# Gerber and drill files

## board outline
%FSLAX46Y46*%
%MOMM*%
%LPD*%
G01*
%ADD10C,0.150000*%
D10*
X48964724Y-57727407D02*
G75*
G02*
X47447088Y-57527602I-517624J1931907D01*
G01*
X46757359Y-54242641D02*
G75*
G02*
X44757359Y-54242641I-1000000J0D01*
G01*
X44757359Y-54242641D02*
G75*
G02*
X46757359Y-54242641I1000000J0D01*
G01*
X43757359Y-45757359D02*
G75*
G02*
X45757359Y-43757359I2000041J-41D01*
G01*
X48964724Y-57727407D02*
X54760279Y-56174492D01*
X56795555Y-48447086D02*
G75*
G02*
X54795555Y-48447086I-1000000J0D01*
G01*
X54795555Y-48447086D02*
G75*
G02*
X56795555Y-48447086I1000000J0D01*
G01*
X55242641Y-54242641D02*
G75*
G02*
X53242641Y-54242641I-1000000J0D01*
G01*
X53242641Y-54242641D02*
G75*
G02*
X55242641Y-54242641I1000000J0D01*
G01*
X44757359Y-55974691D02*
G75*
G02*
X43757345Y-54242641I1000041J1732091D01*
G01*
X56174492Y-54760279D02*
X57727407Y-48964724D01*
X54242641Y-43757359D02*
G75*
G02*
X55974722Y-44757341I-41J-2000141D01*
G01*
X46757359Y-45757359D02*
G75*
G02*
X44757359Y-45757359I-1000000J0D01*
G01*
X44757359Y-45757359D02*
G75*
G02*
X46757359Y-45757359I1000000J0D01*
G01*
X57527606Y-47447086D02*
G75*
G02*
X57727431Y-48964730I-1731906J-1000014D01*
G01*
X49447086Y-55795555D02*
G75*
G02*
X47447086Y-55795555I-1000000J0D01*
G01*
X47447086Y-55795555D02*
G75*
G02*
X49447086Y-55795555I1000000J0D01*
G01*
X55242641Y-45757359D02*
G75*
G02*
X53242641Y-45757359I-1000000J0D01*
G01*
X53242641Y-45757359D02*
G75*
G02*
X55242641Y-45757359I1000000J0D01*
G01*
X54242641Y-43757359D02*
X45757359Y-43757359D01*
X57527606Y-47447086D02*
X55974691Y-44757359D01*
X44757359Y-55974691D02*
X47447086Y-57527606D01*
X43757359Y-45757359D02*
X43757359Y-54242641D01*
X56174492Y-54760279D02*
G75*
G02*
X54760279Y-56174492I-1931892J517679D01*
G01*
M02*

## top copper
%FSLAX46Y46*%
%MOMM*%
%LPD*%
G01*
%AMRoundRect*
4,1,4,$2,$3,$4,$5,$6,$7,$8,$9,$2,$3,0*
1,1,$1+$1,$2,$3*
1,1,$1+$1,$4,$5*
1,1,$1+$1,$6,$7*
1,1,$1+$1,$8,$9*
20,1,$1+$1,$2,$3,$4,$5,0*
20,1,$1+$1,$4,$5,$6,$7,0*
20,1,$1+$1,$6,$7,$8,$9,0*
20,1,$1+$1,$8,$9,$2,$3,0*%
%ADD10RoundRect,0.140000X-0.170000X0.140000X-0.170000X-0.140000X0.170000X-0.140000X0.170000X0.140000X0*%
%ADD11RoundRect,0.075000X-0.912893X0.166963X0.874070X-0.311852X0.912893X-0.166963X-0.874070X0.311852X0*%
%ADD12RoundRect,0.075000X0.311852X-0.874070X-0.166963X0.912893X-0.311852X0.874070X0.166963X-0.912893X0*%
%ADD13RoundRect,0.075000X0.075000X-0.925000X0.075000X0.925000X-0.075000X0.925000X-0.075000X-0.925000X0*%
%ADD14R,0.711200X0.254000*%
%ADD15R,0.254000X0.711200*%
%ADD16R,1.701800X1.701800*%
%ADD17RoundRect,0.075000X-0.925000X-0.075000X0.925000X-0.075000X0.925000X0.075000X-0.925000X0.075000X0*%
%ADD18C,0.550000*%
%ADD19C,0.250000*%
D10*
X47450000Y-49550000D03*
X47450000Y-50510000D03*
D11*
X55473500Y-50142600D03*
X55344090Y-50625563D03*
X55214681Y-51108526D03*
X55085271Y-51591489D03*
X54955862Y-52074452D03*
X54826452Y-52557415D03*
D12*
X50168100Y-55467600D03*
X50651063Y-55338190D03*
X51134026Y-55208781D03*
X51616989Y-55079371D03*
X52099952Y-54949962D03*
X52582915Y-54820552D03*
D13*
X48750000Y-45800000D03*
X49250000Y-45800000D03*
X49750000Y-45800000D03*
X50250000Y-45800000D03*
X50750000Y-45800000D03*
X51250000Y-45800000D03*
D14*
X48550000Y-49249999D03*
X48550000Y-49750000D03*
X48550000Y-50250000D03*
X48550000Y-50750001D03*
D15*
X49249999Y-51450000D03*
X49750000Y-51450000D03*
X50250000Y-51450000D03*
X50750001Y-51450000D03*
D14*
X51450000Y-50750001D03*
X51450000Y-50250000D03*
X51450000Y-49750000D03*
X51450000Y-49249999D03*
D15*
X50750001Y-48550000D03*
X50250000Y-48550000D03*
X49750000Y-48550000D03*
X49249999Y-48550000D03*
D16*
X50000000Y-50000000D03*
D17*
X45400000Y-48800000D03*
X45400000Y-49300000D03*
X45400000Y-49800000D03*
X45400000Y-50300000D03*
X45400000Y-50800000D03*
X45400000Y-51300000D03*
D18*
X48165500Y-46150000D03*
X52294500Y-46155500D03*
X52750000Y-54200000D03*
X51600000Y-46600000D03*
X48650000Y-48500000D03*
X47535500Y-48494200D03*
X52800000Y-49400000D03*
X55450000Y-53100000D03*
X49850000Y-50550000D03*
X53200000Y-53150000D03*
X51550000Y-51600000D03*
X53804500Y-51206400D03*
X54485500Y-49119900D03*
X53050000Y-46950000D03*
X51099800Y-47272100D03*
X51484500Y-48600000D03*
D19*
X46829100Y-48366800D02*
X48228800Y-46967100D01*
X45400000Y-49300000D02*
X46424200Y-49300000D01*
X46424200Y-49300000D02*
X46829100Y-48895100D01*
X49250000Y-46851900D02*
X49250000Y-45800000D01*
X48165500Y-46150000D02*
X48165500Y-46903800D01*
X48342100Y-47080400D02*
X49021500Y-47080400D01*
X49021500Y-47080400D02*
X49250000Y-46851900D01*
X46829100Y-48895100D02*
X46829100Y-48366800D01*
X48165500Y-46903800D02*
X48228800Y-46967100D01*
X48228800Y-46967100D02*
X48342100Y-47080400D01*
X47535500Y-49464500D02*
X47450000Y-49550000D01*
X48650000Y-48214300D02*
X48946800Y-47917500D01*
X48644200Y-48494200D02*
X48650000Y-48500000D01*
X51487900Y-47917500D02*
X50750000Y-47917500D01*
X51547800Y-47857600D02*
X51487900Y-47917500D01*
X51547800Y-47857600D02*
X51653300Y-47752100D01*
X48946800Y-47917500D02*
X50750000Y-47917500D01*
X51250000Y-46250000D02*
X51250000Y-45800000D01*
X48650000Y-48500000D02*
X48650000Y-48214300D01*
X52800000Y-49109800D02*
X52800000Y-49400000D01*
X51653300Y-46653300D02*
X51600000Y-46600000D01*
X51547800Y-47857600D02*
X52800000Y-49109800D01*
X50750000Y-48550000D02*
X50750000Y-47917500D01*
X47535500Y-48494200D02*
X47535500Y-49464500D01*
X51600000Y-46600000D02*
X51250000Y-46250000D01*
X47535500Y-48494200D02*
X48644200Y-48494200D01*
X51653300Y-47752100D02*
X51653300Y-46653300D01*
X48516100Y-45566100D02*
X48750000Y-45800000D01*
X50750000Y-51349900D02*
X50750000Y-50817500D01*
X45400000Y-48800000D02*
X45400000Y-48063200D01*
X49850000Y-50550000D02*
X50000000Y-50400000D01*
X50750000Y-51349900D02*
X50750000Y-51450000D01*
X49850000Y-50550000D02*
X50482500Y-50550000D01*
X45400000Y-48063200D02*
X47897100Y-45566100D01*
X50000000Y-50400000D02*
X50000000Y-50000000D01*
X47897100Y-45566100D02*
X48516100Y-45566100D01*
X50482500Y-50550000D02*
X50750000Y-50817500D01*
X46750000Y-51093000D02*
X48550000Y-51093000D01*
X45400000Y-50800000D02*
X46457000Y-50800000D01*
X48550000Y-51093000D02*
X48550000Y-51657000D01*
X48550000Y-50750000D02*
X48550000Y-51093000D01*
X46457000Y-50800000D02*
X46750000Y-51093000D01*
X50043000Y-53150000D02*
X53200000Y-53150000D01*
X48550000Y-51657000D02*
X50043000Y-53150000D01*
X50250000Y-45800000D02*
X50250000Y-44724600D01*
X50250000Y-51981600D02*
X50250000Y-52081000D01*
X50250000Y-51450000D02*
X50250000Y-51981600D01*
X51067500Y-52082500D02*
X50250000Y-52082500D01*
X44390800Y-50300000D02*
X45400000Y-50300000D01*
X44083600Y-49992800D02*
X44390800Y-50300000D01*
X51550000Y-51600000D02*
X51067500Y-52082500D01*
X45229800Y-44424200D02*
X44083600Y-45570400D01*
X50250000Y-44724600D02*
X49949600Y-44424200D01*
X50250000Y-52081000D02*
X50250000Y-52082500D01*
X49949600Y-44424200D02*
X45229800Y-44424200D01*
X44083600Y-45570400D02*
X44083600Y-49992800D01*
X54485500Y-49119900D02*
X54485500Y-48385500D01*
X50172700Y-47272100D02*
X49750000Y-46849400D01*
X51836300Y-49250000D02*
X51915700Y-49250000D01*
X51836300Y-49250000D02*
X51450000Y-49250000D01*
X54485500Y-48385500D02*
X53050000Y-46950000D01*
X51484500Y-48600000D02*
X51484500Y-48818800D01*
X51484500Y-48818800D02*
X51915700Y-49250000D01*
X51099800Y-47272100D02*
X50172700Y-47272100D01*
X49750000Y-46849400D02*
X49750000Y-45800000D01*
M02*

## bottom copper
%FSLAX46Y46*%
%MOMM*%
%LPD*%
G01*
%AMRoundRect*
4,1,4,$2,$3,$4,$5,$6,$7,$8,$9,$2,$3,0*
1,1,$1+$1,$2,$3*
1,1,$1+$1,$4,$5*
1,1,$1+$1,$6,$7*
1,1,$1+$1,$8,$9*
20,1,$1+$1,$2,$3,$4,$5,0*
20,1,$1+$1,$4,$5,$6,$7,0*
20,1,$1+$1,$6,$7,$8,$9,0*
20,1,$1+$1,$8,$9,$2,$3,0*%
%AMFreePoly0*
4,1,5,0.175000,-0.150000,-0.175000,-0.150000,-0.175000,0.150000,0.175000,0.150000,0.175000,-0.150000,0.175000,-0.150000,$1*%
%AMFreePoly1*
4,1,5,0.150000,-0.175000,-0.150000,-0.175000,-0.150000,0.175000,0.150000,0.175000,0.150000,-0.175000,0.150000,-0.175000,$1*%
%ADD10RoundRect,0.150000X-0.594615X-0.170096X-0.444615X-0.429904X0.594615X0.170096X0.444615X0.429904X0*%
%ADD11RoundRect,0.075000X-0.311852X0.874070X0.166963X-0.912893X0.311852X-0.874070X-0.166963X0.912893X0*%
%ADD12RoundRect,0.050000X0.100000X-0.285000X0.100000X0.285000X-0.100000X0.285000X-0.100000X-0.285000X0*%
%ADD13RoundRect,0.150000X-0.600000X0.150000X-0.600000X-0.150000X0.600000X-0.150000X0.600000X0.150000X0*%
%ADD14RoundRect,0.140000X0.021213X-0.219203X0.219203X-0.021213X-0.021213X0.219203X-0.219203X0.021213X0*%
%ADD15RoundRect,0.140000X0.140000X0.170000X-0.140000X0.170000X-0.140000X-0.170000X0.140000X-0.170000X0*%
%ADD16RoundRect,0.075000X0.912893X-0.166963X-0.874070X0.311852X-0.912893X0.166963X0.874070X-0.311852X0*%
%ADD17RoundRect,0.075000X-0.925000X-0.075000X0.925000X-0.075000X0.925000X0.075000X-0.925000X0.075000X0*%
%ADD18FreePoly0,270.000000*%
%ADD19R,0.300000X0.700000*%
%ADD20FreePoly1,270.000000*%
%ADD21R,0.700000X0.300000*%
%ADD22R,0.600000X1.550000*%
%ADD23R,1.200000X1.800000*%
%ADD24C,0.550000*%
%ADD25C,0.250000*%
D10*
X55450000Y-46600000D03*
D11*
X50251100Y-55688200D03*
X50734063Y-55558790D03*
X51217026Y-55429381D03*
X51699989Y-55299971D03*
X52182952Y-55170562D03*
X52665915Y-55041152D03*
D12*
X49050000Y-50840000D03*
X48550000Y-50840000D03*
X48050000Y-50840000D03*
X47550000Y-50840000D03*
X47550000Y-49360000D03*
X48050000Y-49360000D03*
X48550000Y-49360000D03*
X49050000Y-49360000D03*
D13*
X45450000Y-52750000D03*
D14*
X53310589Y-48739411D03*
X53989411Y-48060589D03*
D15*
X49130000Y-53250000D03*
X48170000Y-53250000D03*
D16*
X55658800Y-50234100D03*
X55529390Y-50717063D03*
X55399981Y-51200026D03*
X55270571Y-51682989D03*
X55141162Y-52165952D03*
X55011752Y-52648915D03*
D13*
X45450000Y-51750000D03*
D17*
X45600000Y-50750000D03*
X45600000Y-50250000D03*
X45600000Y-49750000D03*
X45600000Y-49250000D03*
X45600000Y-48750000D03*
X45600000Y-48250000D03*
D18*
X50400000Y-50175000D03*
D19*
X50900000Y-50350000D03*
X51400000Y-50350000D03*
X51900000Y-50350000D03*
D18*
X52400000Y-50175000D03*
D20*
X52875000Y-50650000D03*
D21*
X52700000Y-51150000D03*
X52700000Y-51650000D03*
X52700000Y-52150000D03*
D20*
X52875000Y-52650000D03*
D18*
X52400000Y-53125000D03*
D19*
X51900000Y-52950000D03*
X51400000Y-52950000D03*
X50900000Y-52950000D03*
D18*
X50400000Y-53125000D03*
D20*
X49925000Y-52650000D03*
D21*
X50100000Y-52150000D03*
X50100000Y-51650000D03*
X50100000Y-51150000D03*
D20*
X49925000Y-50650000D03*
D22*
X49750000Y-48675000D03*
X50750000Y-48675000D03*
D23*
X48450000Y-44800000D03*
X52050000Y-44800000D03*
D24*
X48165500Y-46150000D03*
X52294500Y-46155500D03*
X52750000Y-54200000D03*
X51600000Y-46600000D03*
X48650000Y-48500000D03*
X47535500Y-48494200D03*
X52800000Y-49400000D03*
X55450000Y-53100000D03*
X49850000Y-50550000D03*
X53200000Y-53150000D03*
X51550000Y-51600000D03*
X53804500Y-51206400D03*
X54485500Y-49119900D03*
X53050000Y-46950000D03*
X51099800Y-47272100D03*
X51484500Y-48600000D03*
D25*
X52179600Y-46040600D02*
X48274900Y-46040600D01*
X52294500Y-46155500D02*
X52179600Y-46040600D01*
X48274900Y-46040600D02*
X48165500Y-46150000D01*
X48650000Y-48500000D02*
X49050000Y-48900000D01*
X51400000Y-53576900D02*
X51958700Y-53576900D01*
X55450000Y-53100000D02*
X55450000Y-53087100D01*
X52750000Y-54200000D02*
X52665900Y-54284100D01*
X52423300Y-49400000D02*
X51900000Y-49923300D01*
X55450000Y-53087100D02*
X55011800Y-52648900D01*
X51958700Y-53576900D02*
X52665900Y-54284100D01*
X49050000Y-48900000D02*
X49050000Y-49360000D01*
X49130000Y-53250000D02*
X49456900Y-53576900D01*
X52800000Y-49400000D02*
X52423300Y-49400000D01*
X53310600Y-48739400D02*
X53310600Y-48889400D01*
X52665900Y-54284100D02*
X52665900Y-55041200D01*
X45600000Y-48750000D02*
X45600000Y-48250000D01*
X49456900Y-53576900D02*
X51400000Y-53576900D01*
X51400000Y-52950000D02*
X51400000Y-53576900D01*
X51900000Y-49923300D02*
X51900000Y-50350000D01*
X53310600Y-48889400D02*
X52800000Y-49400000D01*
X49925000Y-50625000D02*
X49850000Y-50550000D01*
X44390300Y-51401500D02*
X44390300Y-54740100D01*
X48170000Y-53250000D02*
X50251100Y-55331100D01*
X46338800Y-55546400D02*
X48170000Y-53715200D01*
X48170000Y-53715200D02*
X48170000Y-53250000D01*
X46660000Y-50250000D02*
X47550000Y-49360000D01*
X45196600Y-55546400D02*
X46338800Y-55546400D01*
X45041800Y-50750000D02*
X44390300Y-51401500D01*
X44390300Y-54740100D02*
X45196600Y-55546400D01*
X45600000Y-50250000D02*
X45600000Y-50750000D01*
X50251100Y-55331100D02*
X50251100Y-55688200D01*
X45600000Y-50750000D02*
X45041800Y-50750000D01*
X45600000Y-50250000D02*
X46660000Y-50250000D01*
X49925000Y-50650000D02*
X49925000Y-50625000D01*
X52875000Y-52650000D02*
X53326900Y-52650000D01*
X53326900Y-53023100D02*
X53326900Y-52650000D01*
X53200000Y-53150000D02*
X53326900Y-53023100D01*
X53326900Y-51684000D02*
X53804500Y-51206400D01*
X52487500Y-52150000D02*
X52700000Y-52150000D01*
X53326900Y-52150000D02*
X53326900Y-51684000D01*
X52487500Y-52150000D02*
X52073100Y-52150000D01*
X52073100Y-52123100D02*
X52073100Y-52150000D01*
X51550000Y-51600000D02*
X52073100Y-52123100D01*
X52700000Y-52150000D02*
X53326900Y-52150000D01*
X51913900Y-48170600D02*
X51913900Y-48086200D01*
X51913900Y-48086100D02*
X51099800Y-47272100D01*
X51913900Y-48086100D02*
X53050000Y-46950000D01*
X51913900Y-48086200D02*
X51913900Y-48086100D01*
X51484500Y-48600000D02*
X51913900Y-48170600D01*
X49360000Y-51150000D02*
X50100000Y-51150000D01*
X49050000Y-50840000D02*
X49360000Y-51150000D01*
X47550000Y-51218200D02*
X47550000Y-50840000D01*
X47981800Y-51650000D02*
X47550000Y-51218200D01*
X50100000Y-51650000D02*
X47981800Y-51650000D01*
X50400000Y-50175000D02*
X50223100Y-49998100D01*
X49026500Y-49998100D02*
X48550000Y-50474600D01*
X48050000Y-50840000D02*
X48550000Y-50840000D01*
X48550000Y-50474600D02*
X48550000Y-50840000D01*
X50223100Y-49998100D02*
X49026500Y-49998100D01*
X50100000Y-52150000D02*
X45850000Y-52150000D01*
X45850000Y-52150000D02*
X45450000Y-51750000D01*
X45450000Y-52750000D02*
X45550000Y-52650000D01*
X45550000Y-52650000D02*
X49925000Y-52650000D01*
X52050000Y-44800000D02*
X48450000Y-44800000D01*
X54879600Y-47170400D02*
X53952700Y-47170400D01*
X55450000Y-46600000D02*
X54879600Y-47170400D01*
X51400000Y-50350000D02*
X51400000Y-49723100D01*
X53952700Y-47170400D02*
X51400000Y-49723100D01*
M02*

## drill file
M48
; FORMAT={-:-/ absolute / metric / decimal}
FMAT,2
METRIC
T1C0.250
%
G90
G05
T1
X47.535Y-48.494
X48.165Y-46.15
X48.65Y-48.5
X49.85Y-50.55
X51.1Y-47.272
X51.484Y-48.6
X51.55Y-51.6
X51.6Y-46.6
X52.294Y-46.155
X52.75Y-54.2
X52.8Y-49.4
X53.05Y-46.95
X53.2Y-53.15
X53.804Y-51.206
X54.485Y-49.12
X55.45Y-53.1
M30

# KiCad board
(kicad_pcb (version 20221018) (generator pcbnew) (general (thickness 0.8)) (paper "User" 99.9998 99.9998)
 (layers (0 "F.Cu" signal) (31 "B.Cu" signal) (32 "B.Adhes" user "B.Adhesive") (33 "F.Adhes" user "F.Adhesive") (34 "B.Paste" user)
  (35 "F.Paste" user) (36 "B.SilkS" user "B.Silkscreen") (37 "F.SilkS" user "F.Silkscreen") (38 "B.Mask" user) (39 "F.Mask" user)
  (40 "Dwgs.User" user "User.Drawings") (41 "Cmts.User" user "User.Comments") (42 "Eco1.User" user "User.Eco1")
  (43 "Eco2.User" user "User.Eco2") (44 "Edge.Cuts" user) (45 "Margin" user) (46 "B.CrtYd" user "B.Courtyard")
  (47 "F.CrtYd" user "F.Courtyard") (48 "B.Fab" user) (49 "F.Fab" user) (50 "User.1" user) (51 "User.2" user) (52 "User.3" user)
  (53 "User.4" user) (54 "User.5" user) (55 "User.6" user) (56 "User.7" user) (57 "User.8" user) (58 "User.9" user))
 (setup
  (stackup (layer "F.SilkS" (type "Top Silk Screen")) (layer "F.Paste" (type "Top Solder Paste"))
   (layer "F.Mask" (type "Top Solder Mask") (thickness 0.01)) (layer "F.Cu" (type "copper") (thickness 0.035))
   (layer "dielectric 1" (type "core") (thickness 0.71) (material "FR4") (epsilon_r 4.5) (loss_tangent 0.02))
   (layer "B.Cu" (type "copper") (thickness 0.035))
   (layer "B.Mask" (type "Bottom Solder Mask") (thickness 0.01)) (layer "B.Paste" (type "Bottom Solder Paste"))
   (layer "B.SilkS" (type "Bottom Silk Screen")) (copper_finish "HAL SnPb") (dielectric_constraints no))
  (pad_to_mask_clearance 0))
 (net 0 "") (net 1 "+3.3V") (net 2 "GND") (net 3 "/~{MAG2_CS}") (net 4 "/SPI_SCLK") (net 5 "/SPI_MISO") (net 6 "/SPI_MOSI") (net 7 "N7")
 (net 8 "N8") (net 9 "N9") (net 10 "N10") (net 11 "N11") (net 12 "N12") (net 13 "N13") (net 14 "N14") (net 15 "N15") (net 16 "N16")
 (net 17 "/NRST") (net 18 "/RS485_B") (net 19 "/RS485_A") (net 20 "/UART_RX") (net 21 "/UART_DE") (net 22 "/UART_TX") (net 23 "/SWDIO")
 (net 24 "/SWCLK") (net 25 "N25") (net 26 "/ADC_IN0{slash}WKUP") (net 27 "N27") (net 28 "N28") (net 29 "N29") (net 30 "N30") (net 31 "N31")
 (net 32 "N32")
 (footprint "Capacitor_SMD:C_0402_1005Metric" (layer "F.Cu") (at 47.45 50.03 -90)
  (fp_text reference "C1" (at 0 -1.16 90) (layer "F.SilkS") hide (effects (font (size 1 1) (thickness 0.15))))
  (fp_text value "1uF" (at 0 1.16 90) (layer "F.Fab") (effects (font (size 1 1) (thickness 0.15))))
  (pad "1" smd roundrect (at -0.48 0 270) (size 0.56 0.62) (layers "F.Cu" "F.Paste" "F.Mask") (roundrect_rratio 0.25) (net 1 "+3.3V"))
  (pad "2" smd roundrect (at 0.48 0 270) (size 0.56 0.62) (layers "F.Cu" "F.Paste" "F.Mask") (roundrect_rratio 0.25) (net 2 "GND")))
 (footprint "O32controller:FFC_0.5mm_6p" (layer "F.Cu") (at 55.4735 50.1426 -15)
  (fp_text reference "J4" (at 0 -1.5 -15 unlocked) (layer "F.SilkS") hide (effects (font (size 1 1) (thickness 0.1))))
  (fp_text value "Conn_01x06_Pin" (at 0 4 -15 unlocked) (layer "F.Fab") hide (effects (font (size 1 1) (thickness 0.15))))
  (pad "1" smd roundrect (at 0 0 345) (size 2 0.3) (layers "F.Cu" "F.Mask") (roundrect_rratio 0.25) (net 2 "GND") (thermal_bridge_angle 45))
  (pad "2" smd roundrect (at 0 0.5 345) (size 2 0.3) (layers "F.Cu" "F.Mask") (roundrect_rratio 0.25) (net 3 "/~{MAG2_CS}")
   (thermal_bridge_angle 45))
  (pad "3" smd roundrect (at 0 1 345) (size 2 0.3) (layers "F.Cu" "F.Mask") (roundrect_rratio 0.25) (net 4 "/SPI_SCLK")
   (thermal_bridge_angle 45))
  (pad "4" smd roundrect (at 0 1.5 345) (size 2 0.3) (layers "F.Cu" "F.Mask") (roundrect_rratio 0.25) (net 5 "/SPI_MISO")
   (thermal_bridge_angle 45))
  (pad "5" smd roundrect (at 0 2 345) (size 2 0.3) (layers "F.Cu" "F.Mask") (roundrect_rratio 0.25) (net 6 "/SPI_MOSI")
   (thermal_bridge_angle 45))
  (pad "6" smd roundrect (at 0 2.5 345) (size 2 0.3) (layers "F.Cu" "F.Mask") (roundrect_rratio 0.25) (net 1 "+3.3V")
   (thermal_bridge_angle 45)))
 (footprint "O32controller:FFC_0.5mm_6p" (layer "F.Cu") (at 50.1681 55.4676 105)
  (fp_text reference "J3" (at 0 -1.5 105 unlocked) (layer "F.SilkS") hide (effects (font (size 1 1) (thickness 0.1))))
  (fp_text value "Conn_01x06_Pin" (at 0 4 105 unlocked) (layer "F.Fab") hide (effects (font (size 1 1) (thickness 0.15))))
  (pad "1" smd roundrect (at 0 0 105) (size 2 0.3) (layers "F.Cu" "F.Mask") (roundrect_rratio 0.25) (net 2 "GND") (thermal_bridge_angle 45))
  (pad "2" smd roundrect (at 0 0.5 105) (size 2 0.3) (layers "F.Cu" "F.Mask") (roundrect_rratio 0.25) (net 3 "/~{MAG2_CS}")
   (thermal_bridge_angle 45))
  (pad "3" smd roundrect (at 0 1 105) (size 2 0.3) (layers "F.Cu" "F.Mask") (roundrect_rratio 0.25) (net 4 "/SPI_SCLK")
   (thermal_bridge_angle 45))
  (pad "4" smd roundrect (at 0 1.5 105) (size 2 0.3) (layers "F.Cu" "F.Mask") (roundrect_rratio 0.25) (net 5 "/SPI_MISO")
   (thermal_bridge_angle 45))
  (pad "5" smd roundrect (at 0 2 105) (size 2 0.3) (layers "F.Cu" "F.Mask") (roundrect_rratio 0.25) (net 6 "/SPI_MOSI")
   (thermal_bridge_angle 45))
  (pad "6" smd roundrect (at 0 2.5 105) (size 2 0.3) (layers "F.Cu" "F.Mask") (roundrect_rratio 0.25) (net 1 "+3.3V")
   (thermal_bridge_angle 45)))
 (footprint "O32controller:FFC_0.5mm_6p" (layer "F.Cu") (at 48.75 45.8 90)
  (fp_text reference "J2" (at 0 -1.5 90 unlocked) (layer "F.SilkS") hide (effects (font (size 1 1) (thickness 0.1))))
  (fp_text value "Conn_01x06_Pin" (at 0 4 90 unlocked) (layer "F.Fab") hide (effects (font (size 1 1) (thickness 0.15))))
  (pad "1" smd roundrect (at 0 0 90) (size 2 0.3) (layers "F.Cu" "F.Mask") (roundrect_rratio 0.25) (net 2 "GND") (thermal_bridge_angle 45))
  (pad "2" smd roundrect (at 0 0.5 90) (size 2 0.3) (layers "F.Cu" "F.Mask") (roundrect_rratio 0.25) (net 3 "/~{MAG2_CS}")
   (thermal_bridge_angle 45))
  (pad "3" smd roundrect (at 0 1 90) (size 2 0.3) (layers "F.Cu" "F.Mask") (roundrect_rratio 0.25) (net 4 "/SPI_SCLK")
   (thermal_bridge_angle 45))
  (pad "4" smd roundrect (at 0 1.5 90) (size 2 0.3) (layers "F.Cu" "F.Mask") (roundrect_rratio 0.25) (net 5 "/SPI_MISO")
   (thermal_bridge_angle 45))
  (pad "5" smd roundrect (at 0 2 90) (size 2 0.3) (layers "F.Cu" "F.Mask") (roundrect_rratio 0.25) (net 6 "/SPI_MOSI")
   (thermal_bridge_angle 45))
  (pad "6" smd roundrect (at 0 2.5 90) (size 2 0.3) (layers "F.Cu" "F.Mask") (roundrect_rratio 0.25) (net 1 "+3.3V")
   (thermal_bridge_angle 45)))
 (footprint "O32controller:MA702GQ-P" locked (layer "F.Cu") (at 50 50)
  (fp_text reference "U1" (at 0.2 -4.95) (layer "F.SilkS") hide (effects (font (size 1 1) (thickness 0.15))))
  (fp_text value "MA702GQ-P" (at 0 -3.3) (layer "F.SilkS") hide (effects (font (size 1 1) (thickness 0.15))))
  (pad "1" smd rect locked (at -1.45 -0.750001) (size 0.7112 0.254) (layers "F.Cu" "F.Paste" "F.Mask") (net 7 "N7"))
  (pad "2" smd rect locked (at -1.45 -0.25) (size 0.7112 0.254) (layers "F.Cu" "F.Paste" "F.Mask") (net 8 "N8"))
  (pad "3" smd rect locked (at -1.45 0.25) (size 0.7112 0.254) (layers "F.Cu" "F.Paste" "F.Mask") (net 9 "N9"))
  (pad "4" smd rect locked (at -1.45 0.750001) (size 0.7112 0.254) (layers "F.Cu" "F.Paste" "F.Mask") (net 6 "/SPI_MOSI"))
  (pad "5" smd rect locked (at -0.750001 1.45 90) (size 0.7112 0.254) (layers "F.Cu" "F.Paste" "F.Mask") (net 3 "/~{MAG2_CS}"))
  (pad "6" smd rect locked (at -0.25 1.45 90) (size 0.7112 0.254) (layers "F.Cu" "F.Paste" "F.Mask") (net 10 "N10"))
  (pad "7" smd rect locked (at 0.25 1.45 90) (size 0.7112 0.254) (layers "F.Cu" "F.Paste" "F.Mask") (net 5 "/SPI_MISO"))
  (pad "8" smd rect locked (at 0.750001 1.45 90) (size 0.7112 0.254) (layers "F.Cu" "F.Paste" "F.Mask") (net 2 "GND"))
  (pad "9" smd rect locked (at 1.45 0.750001) (size 0.7112 0.254) (layers "F.Cu" "F.Paste" "F.Mask") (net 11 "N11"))
  (pad "10" smd rect locked (at 1.45 0.25) (size 0.7112 0.254) (layers "F.Cu" "F.Paste" "F.Mask") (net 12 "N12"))
  (pad "11" smd rect locked (at 1.45 -0.25) (size 0.7112 0.254) (layers "F.Cu" "F.Paste" "F.Mask") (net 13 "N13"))
  (pad "12" smd rect locked (at 1.45 -0.750001) (size 0.7112 0.254) (layers "F.Cu" "F.Paste" "F.Mask") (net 4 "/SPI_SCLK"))
  (pad "13" smd rect locked (at 0.750001 -1.45 90) (size 0.7112 0.254) (layers "F.Cu" "F.Paste" "F.Mask") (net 1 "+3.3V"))
  (pad "14" smd rect locked (at 0.25 -1.45 90) (size 0.7112 0.254) (layers "F.Cu" "F.Paste" "F.Mask") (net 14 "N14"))
  (pad "15" smd rect locked (at -0.25 -1.45 90) (size 0.7112 0.254) (layers "F.Cu" "F.Paste" "F.Mask") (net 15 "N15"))
  (pad "16" smd rect locked (at -0.750001 -1.45 90) (size 0.7112 0.254) (layers "F.Cu" "F.Paste" "F.Mask") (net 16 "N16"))
  (pad "17" smd rect locked (at 0 0) (size 1.7018 1.7018) (layers "F.Cu" "F.Paste" "F.Mask") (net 2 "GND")))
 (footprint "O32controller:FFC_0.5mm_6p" (layer "F.Cu") (at 45.4 48.8)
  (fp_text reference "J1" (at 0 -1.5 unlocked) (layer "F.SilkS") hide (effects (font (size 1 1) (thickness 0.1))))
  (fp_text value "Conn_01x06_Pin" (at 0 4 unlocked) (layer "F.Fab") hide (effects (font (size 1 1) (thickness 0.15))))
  (pad "1" smd roundrect (at 0 0) (size 2 0.3) (layers "F.Cu" "F.Mask") (roundrect_rratio 0.25) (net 2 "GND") (thermal_bridge_angle 45))
  (pad "2" smd roundrect (at 0 0.5) (size 2 0.3) (layers "F.Cu" "F.Mask") (roundrect_rratio 0.25) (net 3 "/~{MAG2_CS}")
   (thermal_bridge_angle 45))
  (pad "3" smd roundrect (at 0 1) (size 2 0.3) (layers "F.Cu" "F.Mask") (roundrect_rratio 0.25) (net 4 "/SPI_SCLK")
   (thermal_bridge_angle 45))
  (pad "4" smd roundrect (at 0 1.5) (size 2 0.3) (layers "F.Cu" "F.Mask") (roundrect_rratio 0.25) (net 5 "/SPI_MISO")
   (thermal_bridge_angle 45))
  (pad "5" smd roundrect (at 0 2) (size 2 0.3) (layers "F.Cu" "F.Mask") (roundrect_rratio 0.25) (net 6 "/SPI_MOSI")
   (thermal_bridge_angle 45))
  (pad "6" smd roundrect (at 0 2.5) (size 2 0.3) (layers "F.Cu" "F.Mask") (roundrect_rratio 0.25) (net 1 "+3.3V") (thermal_bridge_angle 45)))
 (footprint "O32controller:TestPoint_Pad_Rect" (layer "B.Cu") (at 55.45 46.6 -60)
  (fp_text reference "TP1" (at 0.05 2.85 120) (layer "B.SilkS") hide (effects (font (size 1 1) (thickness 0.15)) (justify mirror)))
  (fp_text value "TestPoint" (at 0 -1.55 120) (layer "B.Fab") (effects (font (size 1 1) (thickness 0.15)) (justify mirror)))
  (pad "1" smd roundrect (at 0 0 300) (size 0.6 1.5) (layers "B.Cu" "B.Mask") (roundrect_rratio 0.25) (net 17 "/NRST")))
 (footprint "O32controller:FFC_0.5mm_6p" (layer "B.Cu") (at 50.2511 55.6882 -75)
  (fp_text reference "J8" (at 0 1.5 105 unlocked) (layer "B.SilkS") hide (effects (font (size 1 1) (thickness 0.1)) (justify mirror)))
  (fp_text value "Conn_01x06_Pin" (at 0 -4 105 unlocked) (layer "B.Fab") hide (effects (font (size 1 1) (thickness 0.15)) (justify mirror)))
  (pad "1" smd roundrect (at 0 0 285) (size 2 0.3) (layers "B.Cu" "B.Mask") (roundrect_rratio 0.25) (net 2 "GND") (thermal_bridge_angle 45))
  (pad "2" smd roundrect (at 0 -0.5 285) (size 2 0.3) (layers "B.Cu" "B.Mask") (roundrect_rratio 0.25) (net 2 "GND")
   (thermal_bridge_angle 45))
  (pad "3" smd roundrect (at 0 -1 285) (size 2 0.3) (layers "B.Cu" "B.Mask") (roundrect_rratio 0.25) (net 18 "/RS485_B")
   (thermal_bridge_angle 45))
  (pad "4" smd roundrect (at 0 -1.5 285) (size 2 0.3) (layers "B.Cu" "B.Mask") (roundrect_rratio 0.25) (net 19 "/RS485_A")
   (thermal_bridge_angle 45))
  (pad "5" smd roundrect (at 0 -2 285) (size 2 0.3) (layers "B.Cu" "B.Mask") (roundrect_rratio 0.25) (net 1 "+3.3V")
   (thermal_bridge_angle 45))
  (pad "6" smd roundrect (at 0 -2.5 285) (size 2 0.3) (layers "B.Cu" "B.Mask") (roundrect_rratio 0.25) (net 1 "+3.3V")
   (thermal_bridge_angle 45)))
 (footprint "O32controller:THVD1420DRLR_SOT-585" (layer "B.Cu") (at 48.3 50.1 90)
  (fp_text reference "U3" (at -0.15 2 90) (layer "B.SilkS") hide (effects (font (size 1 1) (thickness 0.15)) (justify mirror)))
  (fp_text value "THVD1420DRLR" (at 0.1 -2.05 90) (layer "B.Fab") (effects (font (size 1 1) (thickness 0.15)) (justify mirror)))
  (pad "1" smd roundrect (at -0.74 0.75 90) (size 0.67 0.3) (layers "B.Cu" "B.Paste" "B.Mask") (roundrect_rratio 0.1666666667)
   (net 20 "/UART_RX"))
  (pad "2" smd roundrect (at -0.74 0.25 90) (size 0.67 0.3) (layers "B.Cu" "B.Paste" "B.Mask") (roundrect_rratio 0.1666666667)
   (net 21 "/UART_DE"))
  (pad "3" smd roundrect (at -0.74 -0.25 90) (size 0.67 0.3) (layers "B.Cu" "B.Paste" "B.Mask") (roundrect_rratio 0.1666666667)
   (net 21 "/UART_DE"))
  (pad "4" smd roundrect (at -0.74 -0.75 90) (size 0.67 0.3) (layers "B.Cu" "B.Paste" "B.Mask") (roundrect_rratio 0.1666666667)
   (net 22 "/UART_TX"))
  (pad "5" smd roundrect (at 0.74 -0.75 90) (size 0.67 0.3) (layers "B.Cu" "B.Paste" "B.Mask") (roundrect_rratio 0.1666666667) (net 2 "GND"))
  (pad "6" smd roundrect (at 0.74 -0.25 90) (size 0.67 0.3) (layers "B.Cu" "B.Paste" "B.Mask") (roundrect_rratio 0.1666666667)
   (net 19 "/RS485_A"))
  (pad "7" smd roundrect (at 0.74 0.25 90) (size 0.67 0.3) (layers "B.Cu" "B.Paste" "B.Mask") (roundrect_rratio 0.1666666667)
   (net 18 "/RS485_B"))
  (pad "8" smd roundrect (at 0.74 0.75 90) (size 0.67 0.3) (layers "B.Cu" "B.Paste" "B.Mask") (roundrect_rratio 0.1666666667)
   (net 1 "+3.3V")))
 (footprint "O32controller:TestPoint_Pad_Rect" (layer "B.Cu") (at 45.45 52.75 -90)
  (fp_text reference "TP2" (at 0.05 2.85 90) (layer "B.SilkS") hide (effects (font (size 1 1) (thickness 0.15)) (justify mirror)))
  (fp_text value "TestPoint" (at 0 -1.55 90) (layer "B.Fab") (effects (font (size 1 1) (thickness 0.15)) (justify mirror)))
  (pad "1" smd roundrect (at 0 0 270) (size 0.6 1.5) (layers "B.Cu" "B.Mask") (roundrect_rratio 0.25) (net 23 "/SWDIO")))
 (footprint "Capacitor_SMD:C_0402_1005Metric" (layer "B.Cu") (at 53.65 48.4 45)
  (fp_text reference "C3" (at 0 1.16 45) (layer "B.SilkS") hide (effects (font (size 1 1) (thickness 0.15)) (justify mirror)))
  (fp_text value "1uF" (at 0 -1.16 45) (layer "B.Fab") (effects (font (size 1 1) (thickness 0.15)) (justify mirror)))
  (pad "1" smd roundrect (at -0.48 0 45) (size 0.56 0.62) (layers "B.Cu" "B.Paste" "B.Mask") (roundrect_rratio 0.25) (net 1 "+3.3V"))
  (pad "2" smd roundrect (at 0.48 0 45) (size 0.56 0.62) (layers "B.Cu" "B.Paste" "B.Mask") (roundrect_rratio 0.25) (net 2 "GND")))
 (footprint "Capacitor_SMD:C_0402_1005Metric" (layer "B.Cu") (at 48.65 53.25 180)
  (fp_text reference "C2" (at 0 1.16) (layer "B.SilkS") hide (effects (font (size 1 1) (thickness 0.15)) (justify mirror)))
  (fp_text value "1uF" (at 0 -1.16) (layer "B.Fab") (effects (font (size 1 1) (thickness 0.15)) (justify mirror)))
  (pad "1" smd roundrect (at -0.48 0 180) (size 0.56 0.62) (layers "B.Cu" "B.Paste" "B.Mask") (roundrect_rratio 0.25) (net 1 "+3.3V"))
  (pad "2" smd roundrect (at 0.48 0 180) (size 0.56 0.62) (layers "B.Cu" "B.Paste" "B.Mask") (roundrect_rratio 0.25) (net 2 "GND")))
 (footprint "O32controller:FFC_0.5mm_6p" (layer "B.Cu") (at 55.6588 50.2341 165)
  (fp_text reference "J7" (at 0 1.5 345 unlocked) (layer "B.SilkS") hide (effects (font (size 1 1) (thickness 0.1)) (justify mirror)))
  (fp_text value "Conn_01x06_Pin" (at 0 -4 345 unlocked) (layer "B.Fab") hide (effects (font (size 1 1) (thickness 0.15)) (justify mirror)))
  (pad "1" smd roundrect (at 0 0 165) (size 2 0.3) (layers "B.Cu" "B.Mask") (roundrect_rratio 0.25) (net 2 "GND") (thermal_bridge_angle 45))
  (pad "2" smd roundrect (at 0 -0.5 165) (size 2 0.3) (layers "B.Cu" "B.Mask") (roundrect_rratio 0.25) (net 2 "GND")
   (thermal_bridge_angle 45))
  (pad "3" smd roundrect (at 0 -1 165) (size 2 0.3) (layers "B.Cu" "B.Mask") (roundrect_rratio 0.25) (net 18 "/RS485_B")
   (thermal_bridge_angle 45))
  (pad "4" smd roundrect (at 0 -1.5 165) (size 2 0.3) (layers "B.Cu" "B.Mask") (roundrect_rratio 0.25) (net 19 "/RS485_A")
   (thermal_bridge_angle 45))
  (pad "5" smd roundrect (at 0 -2 165) (size 2 0.3) (layers "B.Cu" "B.Mask") (roundrect_rratio 0.25) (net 1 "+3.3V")
   (thermal_bridge_angle 45))
  (pad "6" smd roundrect (at 0 -2.5 165) (size 2 0.3) (layers "B.Cu" "B.Mask") (roundrect_rratio 0.25) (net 1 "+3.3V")
   (thermal_bridge_angle 45)))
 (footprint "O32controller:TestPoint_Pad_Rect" (layer "B.Cu") (at 45.45 51.75 -90)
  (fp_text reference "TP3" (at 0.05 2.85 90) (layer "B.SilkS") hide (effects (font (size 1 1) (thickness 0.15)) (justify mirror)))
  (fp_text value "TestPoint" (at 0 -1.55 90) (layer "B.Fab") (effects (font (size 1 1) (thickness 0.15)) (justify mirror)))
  (pad "1" smd roundrect (at 0 0 270) (size 0.6 1.5) (layers "B.Cu" "B.Mask") (roundrect_rratio 0.25) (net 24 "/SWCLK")))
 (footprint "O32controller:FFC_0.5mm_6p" (layer "B.Cu") (at 45.6 50.75)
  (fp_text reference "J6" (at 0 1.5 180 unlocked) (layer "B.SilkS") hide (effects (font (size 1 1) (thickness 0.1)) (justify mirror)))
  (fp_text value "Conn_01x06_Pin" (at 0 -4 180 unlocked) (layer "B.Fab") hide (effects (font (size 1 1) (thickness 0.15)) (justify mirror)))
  (pad "1" smd roundrect (at 0 0) (size 2 0.3) (layers "B.Cu" "B.Mask") (roundrect_rratio 0.25) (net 2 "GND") (thermal_bridge_angle 45))
  (pad "2" smd roundrect (at 0 -0.5) (size 2 0.3) (layers "B.Cu" "B.Mask") (roundrect_rratio 0.25) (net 2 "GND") (thermal_bridge_angle 45))
  (pad "3" smd roundrect (at 0 -1) (size 2 0.3) (layers "B.Cu" "B.Mask") (roundrect_rratio 0.25) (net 18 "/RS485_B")
   (thermal_bridge_angle 45))
  (pad "4" smd roundrect (at 0 -1.5) (size 2 0.3) (layers "B.Cu" "B.Mask") (roundrect_rratio 0.25) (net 19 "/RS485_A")
   (thermal_bridge_angle 45))
  (pad "5" smd roundrect (at 0 -2) (size 2 0.3) (layers "B.Cu" "B.Mask") (roundrect_rratio 0.25) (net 1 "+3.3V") (thermal_bridge_angle 45))
  (pad "6" smd roundrect (at 0 -2.5) (size 2 0.3) (layers "B.Cu" "B.Mask") (roundrect_rratio 0.25) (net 1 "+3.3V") (thermal_bridge_angle 45)))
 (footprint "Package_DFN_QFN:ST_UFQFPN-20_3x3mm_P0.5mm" (layer "B.Cu") (at 51.4 51.65 -90)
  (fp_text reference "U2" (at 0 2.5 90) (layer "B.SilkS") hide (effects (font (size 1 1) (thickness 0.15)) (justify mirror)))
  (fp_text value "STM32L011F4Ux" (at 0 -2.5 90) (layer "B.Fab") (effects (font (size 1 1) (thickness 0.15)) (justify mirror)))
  (pad "1" smd custom (at -1.475 1 270) (size 0.35 0.3) (layers "B.Cu" "B.Paste" "B.Mask") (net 21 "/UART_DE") (zone_connect 2)
   (thermal_bridge_angle 45) (options (clearance outline) (anchor rect)) (primitives))
  (pad "2" smd rect (at -1.3 0.5 270) (size 0.7 0.3) (layers "B.Cu" "B.Paste" "B.Mask") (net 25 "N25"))
  (pad "3" smd rect (at -1.3 0 270) (size 0.7 0.3) (layers "B.Cu" "B.Paste" "B.Mask") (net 17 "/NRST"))
  (pad "4" smd rect (at -1.3 -0.5 270) (size 0.7 0.3) (layers "B.Cu" "B.Paste" "B.Mask") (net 1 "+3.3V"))
  (pad "5" smd custom (at -1.475 -1 270) (size 0.35 0.3) (layers "B.Cu" "B.Paste" "B.Mask") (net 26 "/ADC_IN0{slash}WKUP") (zone_connect 2)
   (thermal_bridge_angle 45) (options (clearance outline) (anchor rect)) (primitives))
  (pad "6" smd custom (at -1 -1.475 270) (size 0.3 0.35) (layers "B.Cu" "B.Paste" "B.Mask") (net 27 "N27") (zone_connect 2)
   (thermal_bridge_angle 45) (options (clearance outline) (anchor rect)) (primitives))
  (pad "7" smd rect (at -0.5 -1.3 270) (size 0.3 0.7) (layers "B.Cu" "B.Paste" "B.Mask") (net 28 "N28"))
  (pad "8" smd rect (at 0 -1.3 270) (size 0.3 0.7) (layers "B.Cu" "B.Paste" "B.Mask") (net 4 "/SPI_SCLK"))
  (pad "9" smd rect (at 0.5 -1.3 270) (size 0.3 0.7) (layers "B.Cu" "B.Paste" "B.Mask") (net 5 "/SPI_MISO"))
  (pad "10" smd custom (at 1 -1.475 270) (size 0.3 0.35) (layers "B.Cu" "B.Paste" "B.Mask") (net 6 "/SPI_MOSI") (zone_connect 2)
   (thermal_bridge_angle 45) (options (clearance outline) (anchor rect)) (primitives))
  (pad "11" smd custom (at 1.475 -1 270) (size 0.35 0.3) (layers "B.Cu" "B.Paste" "B.Mask") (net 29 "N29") (zone_connect 2)
   (thermal_bridge_angle 45) (options (clearance outline) (anchor rect)) (primitives))
  (pad "12" smd rect (at 1.3 -0.5 270) (size 0.7 0.3) (layers "B.Cu" "B.Paste" "B.Mask") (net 2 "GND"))
  (pad "13" smd rect (at 1.3 0 270) (size 0.7 0.3) (layers "B.Cu" "B.Paste" "B.Mask") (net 1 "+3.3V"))
  (pad "14" smd rect (at 1.3 0.5 270) (size 0.7 0.3) (layers "B.Cu" "B.Paste" "B.Mask") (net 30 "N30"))
  (pad "15" smd custom (at 1.475 1 270) (size 0.35 0.3) (layers "B.Cu" "B.Paste" "B.Mask") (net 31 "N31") (zone_connect 2)
   (thermal_bridge_angle 45) (options (clearance outline) (anchor rect)) (primitives))
  (pad "16" smd custom (at 1 1.475 270) (size 0.3 0.35) (layers "B.Cu" "B.Paste" "B.Mask") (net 23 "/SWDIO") (zone_connect 2)
   (thermal_bridge_angle 45) (options (clearance outline) (anchor rect)) (primitives))
  (pad "17" smd rect (at 0.5 1.3 270) (size 0.3 0.7) (layers "B.Cu" "B.Paste" "B.Mask") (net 24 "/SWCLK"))
  (pad "18" smd rect (at 0 1.3 270) (size 0.3 0.7) (layers "B.Cu" "B.Paste" "B.Mask") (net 22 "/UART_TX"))
  (pad "19" smd rect (at -0.5 1.3 270) (size 0.3 0.7) (layers "B.Cu" "B.Paste" "B.Mask") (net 20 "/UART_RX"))
  (pad "20" smd custom (at -1 1.475 270) (size 0.3 0.35) (layers "B.Cu" "B.Paste" "B.Mask") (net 2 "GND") (zone_connect 2)
   (thermal_bridge_angle 45) (options (clearance outline) (anchor rect)) (primitives)))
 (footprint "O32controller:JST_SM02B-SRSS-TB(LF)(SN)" (layer "B.Cu") (at 50.25 46.7)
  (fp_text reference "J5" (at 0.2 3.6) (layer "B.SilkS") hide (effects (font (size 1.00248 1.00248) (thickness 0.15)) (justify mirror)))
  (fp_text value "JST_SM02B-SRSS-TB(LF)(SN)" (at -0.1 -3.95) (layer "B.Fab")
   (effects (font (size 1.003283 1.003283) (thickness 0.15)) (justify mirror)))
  (pad "1" smd rect (at -0.5 1.975 270) (size 1.55 0.6) (layers "B.Cu" "B.Paste" "B.Mask") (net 19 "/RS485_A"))
  (pad "2" smd rect (at 0.5 1.975 270) (size 1.55 0.6) (layers "B.Cu" "B.Paste" "B.Mask") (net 18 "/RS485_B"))
  (pad "S1" smd rect (at -1.8 -1.9 270) (size 1.8 1.2) (layers "B.Cu" "B.Paste" "B.Mask") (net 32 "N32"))
  (pad "S2" smd rect (at 1.8 -1.9 270) (size 1.8 1.2) (layers "B.Cu" "B.Paste" "B.Mask") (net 32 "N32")))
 (gr_arc (start 48.964724 57.727407) (mid 48.186036 57.778441) (end 47.447086 57.527606) (stroke (width 0.15) (type solid))
  (layer "Edge.Cuts"))
 (gr_circle (center 45.757359 54.242641) (end 46.757359 54.242641) (stroke (width 0.15) (type solid)) (fill none) (layer "Edge.Cuts"))
 (gr_arc (start 43.757359 45.757359) (mid 44.343157 44.343157) (end 45.757359 43.757359) (stroke (width 0.15) (type solid))
  (layer "Edge.Cuts"))
 (gr_line (start 48.964724 57.727407) (end 54.760279 56.174492) (stroke (width 0.15) (type solid)) (layer "Edge.Cuts"))
 (gr_circle (center 55.795555 48.447086) (end 56.795555 48.447086) (stroke (width 0.15) (type solid)) (fill none) (layer "Edge.Cuts"))
 (gr_circle (center 54.242641 54.242641) (end 55.242641 54.242641) (stroke (width 0.15) (type solid)) (fill none) (layer "Edge.Cuts"))
 (gr_arc (start 44.757359 55.974691) (mid 44.025308 55.242639) (end 43.757359 54.242641) (stroke (width 0.15) (type solid))
  (layer "Edge.Cuts"))
 (gr_line (start 56.174492 54.760279) (end 57.727407 48.964724) (stroke (width 0.15) (type solid)) (layer "Edge.Cuts"))
 (gr_arc (start 54.242641 43.757359) (mid 55.242632 44.02532) (end 55.974691 44.757359) (stroke (width 0.15) (type solid))
  (layer "Edge.Cuts"))
 (gr_circle (center 45.757359 45.757359) (end 46.757359 45.757359) (stroke (width 0.15) (type solid)) (fill none) (layer "Edge.Cuts"))
 (gr_arc (start 57.527606 47.447086) (mid 57.778456 48.186034) (end 57.727407 48.964724) (stroke (width 0.15) (type solid))
  (layer "Edge.Cuts"))
 (gr_circle (center 48.447086 55.795555) (end 49.447086 55.795555) (stroke (width 0.15) (type solid)) (fill none) (layer "Edge.Cuts"))
 (gr_circle (center 54.242641 45.757359) (end 55.242641 45.757359) (stroke (width 0.15) (type solid)) (fill none) (layer "Edge.Cuts"))
 (gr_line (start 54.242641 43.757359) (end 45.757359 43.757359) (stroke (width 0.15) (type solid)) (layer "Edge.Cuts"))
 (gr_line (start 57.527606 47.447086) (end 55.974691 44.757359) (stroke (width 0.15) (type solid)) (layer "Edge.Cuts"))
 (gr_line (start 44.757359 55.974691) (end 47.447086 57.527606) (stroke (width 0.15) (type solid)) (layer "Edge.Cuts"))
 (gr_line (start 43.757359 45.757359) (end 43.757359 54.242641) (stroke (width 0.15) (type solid)) (layer "Edge.Cuts"))
 (gr_arc (start 56.174492 54.760279) (mid 55.656849 55.656849) (end 54.760279 56.174492) (stroke (width 0.15) (type solid))
  (layer "Edge.Cuts"))
 (segment (start 46.8291 48.3668) (end 48.2288 46.9671) (width 0.25) (layer "F.Cu") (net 3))
 (segment (start 45.4 49.3) (end 46.4242 49.3) (width 0.25) (layer "F.Cu") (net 3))
 (segment (start 46.4242 49.3) (end 46.8291 48.8951) (width 0.25) (layer "F.Cu") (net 3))
 (segment (start 49.25 46.8519) (end 49.25 45.8) (width 0.25) (layer "F.Cu") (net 3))
 (segment (start 48.1655 46.15) (end 48.1655 46.9038) (width 0.25) (layer "F.Cu") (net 3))
 (segment (start 48.3421 47.0804) (end 49.0215 47.0804) (width 0.25) (layer "F.Cu") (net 3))
 (segment (start 49.0215 47.0804) (end 49.25 46.8519) (width 0.25) (layer "F.Cu") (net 3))
 (segment (start 46.8291 48.8951) (end 46.8291 48.3668) (width 0.25) (layer "F.Cu") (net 3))
 (segment (start 48.1655 46.9038) (end 48.2288 46.9671) (width 0.25) (layer "F.Cu") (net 3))
 (segment (start 48.2288 46.9671) (end 48.3421 47.0804) (width 0.25) (layer "F.Cu") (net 3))
 (via (at 48.1655 46.15) (size 0.55) (drill 0.25) (layers "F.Cu" "B.Cu") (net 3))
 (via (at 52.2945 46.1555) (size 0.55) (drill 0.25) (layers "F.Cu" "B.Cu") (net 3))
 (segment (start 52.1796 46.0406) (end 48.2749 46.0406) (width 0.25) (layer "B.Cu") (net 3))
 (segment (start 52.2945 46.1555) (end 52.1796 46.0406) (width 0.25) (layer "B.Cu") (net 3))
 (segment (start 48.2749 46.0406) (end 48.1655 46.15) (width 0.25) (layer "B.Cu") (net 3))
 (segment (start 47.5355 49.4645) (end 47.45 49.55) (width 0.25) (layer "F.Cu") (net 1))
 (segment (start 48.65 48.2143) (end 48.9468 47.9175) (width 0.25) (layer "F.Cu") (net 1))
 (segment (start 48.6442 48.4942) (end 48.65 48.5) (width 0.25) (layer "F.Cu") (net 1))
 (segment (start 51.4879 47.9175) (end 50.75 47.9175) (width 0.25) (layer "F.Cu") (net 1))
 (segment (start 51.5478 47.8576) (end 51.4879 47.9175) (width 0.25) (layer "F.Cu") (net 1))
 (segment (start 51.5478 47.8576) (end 51.6533 47.7521) (width 0.25) (layer "F.Cu") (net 1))
 (segment (start 48.9468 47.9175) (end 50.75 47.9175) (width 0.25) (layer "F.Cu") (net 1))
 (segment (start 51.25 46.25) (end 51.25 45.8) (width 0.25) (layer "F.Cu") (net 1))
 (segment (start 48.65 48.5) (end 48.65 48.2143) (width 0.25) (layer "F.Cu") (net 1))
 (segment (start 52.8 49.1098) (end 52.8 49.4) (width 0.25) (layer "F.Cu") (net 1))
 (segment (start 51.6533 46.6533) (end 51.6 46.6) (width 0.25) (layer "F.Cu") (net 1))
 (segment (start 51.5478 47.8576) (end 52.8 49.1098) (width 0.25) (layer "F.Cu") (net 1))
 (segment (start 50.75 48.55) (end 50.75 47.9175) (width 0.25) (layer "F.Cu") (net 1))
 (segment (start 47.5355 48.4942) (end 47.5355 49.4645) (width 0.25) (layer "F.Cu") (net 1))
 (segment (start 51.6 46.6) (end 51.25 46.25) (width 0.25) (layer "F.Cu") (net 1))
 (segment (start 47.5355 48.4942) (end 48.6442 48.4942) (width 0.25) (layer "F.Cu") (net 1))
 (segment (start 51.6533 47.7521) (end 51.6533 46.6533) (width 0.25) (layer "F.Cu") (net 1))
 (via (at 52.75 54.2) (size 0.55) (drill 0.25) (layers "F.Cu" "B.Cu") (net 1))
 (via (at 51.6 46.6) (size 0.55) (drill 0.25) (layers "F.Cu" "B.Cu") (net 1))
 (via (at 48.65 48.5) (size 0.55) (drill 0.25) (layers "F.Cu" "B.Cu") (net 1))
 (via (at 47.5355 48.4942) (size 0.55) (drill 0.25) (layers "F.Cu" "B.Cu") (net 1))
 (via (at 52.8 49.4) (size 0.55) (drill 0.25) (layers "F.Cu" "B.Cu") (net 1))
 (via (at 55.45 53.1) (size 0.55) (drill 0.25) (layers "F.Cu" "B.Cu") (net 1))
 (segment (start 48.65 48.5) (end 49.05 48.9) (width 0.25) (layer "B.Cu") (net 1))
 (segment (start 51.4 53.5769) (end 51.9587 53.5769) (width 0.25) (layer "B.Cu") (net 1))
 (segment (start 55.45 53.1) (end 55.45 53.0871) (width 0.25) (layer "B.Cu") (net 1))
 (segment (start 52.75 54.2) (end 52.6659 54.2841) (width 0.25) (layer "B.Cu") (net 1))
 (segment (start 52.4233 49.4) (end 51.9 49.9233) (width 0.25) (layer "B.Cu") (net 1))
 (segment (start 55.45 53.0871) (end 55.0118 52.6489) (width 0.25) (layer "B.Cu") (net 1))
 (segment (start 51.9587 53.5769) (end 52.6659 54.2841) (width 0.25) (layer "B.Cu") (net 1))
 (segment (start 49.05 48.9) (end 49.05 49.36) (width 0.25) (layer "B.Cu") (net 1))
 (segment (start 49.13 53.25) (end 49.4569 53.5769) (width 0.25) (layer "B.Cu") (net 1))
 (segment (start 52.8 49.4) (end 52.4233 49.4) (width 0.25) (layer "B.Cu") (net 1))
 (segment (start 53.3106 48.7394) (end 53.3106 48.8894) (width 0.25) (layer "B.Cu") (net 1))
 (segment (start 52.6659 54.2841) (end 52.6659 55.0412) (width 0.25) (layer "B.Cu") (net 1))
 (segment (start 45.6 48.75) (end 45.6 48.25) (width 0.25) (layer "B.Cu") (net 1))
 (segment (start 49.4569 53.5769) (end 51.4 53.5769) (width 0.25) (layer "B.Cu") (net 1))
 (segment (start 51.4 52.95) (end 51.4 53.5769) (width 0.25) (layer "B.Cu") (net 1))
 (segment (start 51.9 49.9233) (end 51.9 50.35) (width 0.25) (layer "B.Cu") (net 1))
 (segment (start 53.3106 48.8894) (end 52.8 49.4) (width 0.25) (layer "B.Cu") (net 1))
 (segment (start 48.5161 45.5661) (end 48.75 45.8) (width 0.25) (layer "F.Cu") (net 2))
 (segment (start 50.75 51.3499) (end 50.75 50.8175) (width 0.25) (layer "F.Cu") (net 2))
 (segment (start 45.4 48.8) (end 45.4 48.0632) (width 0.25) (layer "F.Cu") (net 2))
 (segment (start 49.85 50.55) (end 50 50.4) (width 0.25) (layer "F.Cu") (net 2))
 (segment (start 50.75 51.3499) (end 50.75 51.45) (width 0.25) (layer "F.Cu") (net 2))
 (segment (start 49.85 50.55) (end 50.4825 50.55) (width 0.25) (layer "F.Cu") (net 2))
 (segment (start 45.4 48.0632) (end 47.8971 45.5661) (width 0.25) (layer "F.Cu") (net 2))
 (segment (start 50 50.4) (end 50 50) (width 0.25) (layer "F.Cu") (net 2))
 (segment (start 47.8971 45.5661) (end 48.5161 45.5661) (width 0.25) (layer "F.Cu") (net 2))
 (segment (start 50.4825 50.55) (end 50.75 50.8175) (width 0.25) (layer "F.Cu") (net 2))
 (via (at 49.85 50.55) (size 0.55) (drill 0.25) (layers "F.Cu" "B.Cu") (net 2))
 (segment (start 49.925 50.625) (end 49.85 50.55) (width 0.25) (layer "B.Cu") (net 2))
 (segment (start 44.3903 51.4015) (end 44.3903 54.7401) (width 0.25) (layer "B.Cu") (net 2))
 (segment (start 48.17 53.25) (end 50.2511 55.3311) (width 0.25) (layer "B.Cu") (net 2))
 (segment (start 46.3388 55.5464) (end 48.17 53.7152) (width 0.25) (layer "B.Cu") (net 2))
 (segment (start 48.17 53.7152) (end 48.17 53.25) (width 0.25) (layer "B.Cu") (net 2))
 (segment (start 46.66 50.25) (end 47.55 49.36) (width 0.25) (layer "B.Cu") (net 2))
 (segment (start 45.1966 55.5464) (end 46.3388 55.5464) (width 0.25) (layer "B.Cu") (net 2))
 (segment (start 45.0418 50.75) (end 44.3903 51.4015) (width 0.25) (layer "B.Cu") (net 2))
 (segment (start 44.3903 54.7401) (end 45.1966 55.5464) (width 0.25) (layer "B.Cu") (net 2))
 (segment (start 45.6 50.25) (end 45.6 50.75) (width 0.25) (layer "B.Cu") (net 2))
 (segment (start 50.2511 55.3311) (end 50.2511 55.6882) (width 0.25) (layer "B.Cu") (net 2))
 (segment (start 45.6 50.75) (end 45.0418 50.75) (width 0.25) (layer "B.Cu") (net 2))
 (segment (start 45.6 50.25) (end 46.66 50.25) (width 0.25) (layer "B.Cu") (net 2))
 (segment (start 49.925 50.65) (end 49.925 50.625) (width 0.25) (layer "B.Cu") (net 2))
 (segment (start 46.75 51.093) (end 48.55 51.093) (width 0.25) (layer "F.Cu") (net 6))
 (segment (start 45.4 50.8) (end 46.457 50.8) (width 0.25) (layer "F.Cu") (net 6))
 (segment (start 48.55 51.093) (end 48.55 51.657) (width 0.25) (layer "F.Cu") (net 6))
 (segment (start 48.55 50.75) (end 48.55 51.093) (width 0.25) (layer "F.Cu") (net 6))
 (segment (start 46.457 50.8) (end 46.75 51.093) (width 0.25) (layer "F.Cu") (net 6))
 (segment (start 50.043 53.15) (end 53.2 53.15) (width 0.25) (layer "F.Cu") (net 6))
 (segment (start 48.55 51.657) (end 50.043 53.15) (width 0.25) (layer "F.Cu") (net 6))
 (via (at 53.2 53.15) (size 0.55) (drill 0.25) (layers "F.Cu" "B.Cu") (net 6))
 (segment (start 52.875 52.65) (end 53.3269 52.65) (width 0.25) (layer "B.Cu") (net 6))
 (segment (start 53.3269 53.0231) (end 53.3269 52.65) (width 0.25) (layer "B.Cu") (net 6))
 (segment (start 53.2 53.15) (end 53.3269 53.0231) (width 0.25) (layer "B.Cu") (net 6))
 (segment (start 50.25 45.8) (end 50.25 44.7246) (width 0.25) (layer "F.Cu") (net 5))
 (segment (start 50.25 51.9816) (end 50.25 52.081) (width 0.25) (layer "F.Cu") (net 5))
 (segment (start 50.25 51.45) (end 50.25 51.9816) (width 0.25) (layer "F.Cu") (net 5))
 (segment (start 51.0675 52.0825) (end 50.25 52.0825) (width 0.25) (layer "F.Cu") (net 5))
 (segment (start 44.3908 50.3) (end 45.4 50.3) (width 0.25) (layer "F.Cu") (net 5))
 (segment (start 44.0836 49.9928) (end 44.3908 50.3) (width 0.25) (layer "F.Cu") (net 5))
 (segment (start 51.55 51.6) (end 51.0675 52.0825) (width 0.25) (layer "F.Cu") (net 5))
 (segment (start 45.2298 44.4242) (end 44.0836 45.5704) (width 0.25) (layer "F.Cu") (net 5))
 (segment (start 50.25 44.7246) (end 49.9496 44.4242) (width 0.25) (layer "F.Cu") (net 5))
 (segment (start 50.25 52.081) (end 50.25 52.0825) (width 0.25) (layer "F.Cu") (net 5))
 (segment (start 49.9496 44.4242) (end 45.2298 44.4242) (width 0.25) (layer "F.Cu") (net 5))
 (segment (start 44.0836 45.5704) (end 44.0836 49.9928) (width 0.25) (layer "F.Cu") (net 5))
 (via (at 51.55 51.6) (size 0.55) (drill 0.25) (layers "F.Cu" "B.Cu") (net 5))
 (via (at 53.8045 51.2064) (size 0.55) (drill 0.25) (layers "F.Cu" "B.Cu") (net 5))
 (segment (start 53.3269 51.684) (end 53.8045 51.2064) (width 0.25) (layer "B.Cu") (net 5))
 (segment (start 52.4875 52.15) (end 52.7 52.15) (width 0.25) (layer "B.Cu") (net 5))
 (segment (start 53.3269 52.15) (end 53.3269 51.684) (width 0.25) (layer "B.Cu") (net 5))
 (segment (start 52.4875 52.15) (end 52.0731 52.15) (width 0.25) (layer "B.Cu") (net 5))
 (segment (start 52.0731 52.1231) (end 52.0731 52.15) (width 0.25) (layer "B.Cu") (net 5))
 (segment (start 51.55 51.6) (end 52.0731 52.1231) (width 0.25) (layer "B.Cu") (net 5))
 (segment (start 52.7 52.15) (end 53.3269 52.15) (width 0.25) (layer "B.Cu") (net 5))
 (segment (start 54.4855 49.1199) (end 54.4855 48.3855) (width 0.25) (layer "F.Cu") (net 4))
 (segment (start 50.1727 47.2721) (end 49.75 46.8494) (width 0.25) (layer "F.Cu") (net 4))
 (segment (start 51.8363 49.25) (end 51.9157 49.25) (width 0.25) (layer "F.Cu") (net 4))
 (segment (start 51.8363 49.25) (end 51.45 49.25) (width 0.25) (layer "F.Cu") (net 4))
 (segment (start 54.4855 48.3855) (end 53.05 46.95) (width 0.25) (layer "F.Cu") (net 4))
 (segment (start 51.4845 48.6) (end 51.4845 48.8188) (width 0.25) (layer "F.Cu") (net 4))
 (segment (start 51.4845 48.8188) (end 51.9157 49.25) (width 0.25) (layer "F.Cu") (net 4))
 (segment (start 51.0998 47.2721) (end 50.1727 47.2721) (width 0.25) (layer "F.Cu") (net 4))
 (segment (start 49.75 46.8494) (end 49.75 45.8) (width 0.25) (layer "F.Cu") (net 4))
 (via (at 54.4855 49.1199) (size 0.55) (drill 0.25) (layers "F.Cu" "B.Cu") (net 4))
 (via (at 53.05 46.95) (size 0.55) (drill 0.25) (layers "F.Cu" "B.Cu") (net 4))
 (via (at 51.0998 47.2721) (size 0.55) (drill 0.25) (layers "F.Cu" "B.Cu") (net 4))
 (via (at 51.4845 48.6) (size 0.55) (drill 0.25) (layers "F.Cu" "B.Cu") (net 4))
 (segment (start 51.9139 48.1706) (end 51.9139 48.0862) (width 0.25) (layer "B.Cu") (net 4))
 (segment (start 51.9139 48.0861) (end 51.0998 47.2721) (width 0.25) (layer "B.Cu") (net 4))
 (segment (start 51.9139 48.0861) (end 53.05 46.95) (width 0.25) (layer "B.Cu") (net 4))
 (segment (start 51.9139 48.0862) (end 51.9139 48.0861) (width 0.25) (layer "B.Cu") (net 4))
 (segment (start 51.4845 48.6) (end 51.9139 48.1706) (width 0.25) (layer "B.Cu") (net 4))
 (segment (start 49.36 51.15) (end 50.1 51.15) (width 0.25) (layer "B.Cu") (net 20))
 (segment (start 49.05 50.84) (end 49.36 51.15) (width 0.25) (layer "B.Cu") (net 20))
 (segment (start 47.55 51.2182) (end 47.55 50.84) (width 0.25) (layer "B.Cu") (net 22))
 (segment (start 47.9818 51.65) (end 47.55 51.2182) (width 0.25) (layer "B.Cu") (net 22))
 (segment (start 50.1 51.65) (end 47.9818 51.65) (width 0.25) (layer "B.Cu") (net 22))
 (segment (start 50.4 50.175) (end 50.2231 49.9981) (width 0.25) (layer "B.Cu") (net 21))
 (segment (start 49.0265 49.9981) (end 48.55 50.4746) (width 0.25) (layer "B.Cu") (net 21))
 (segment (start 48.05 50.84) (end 48.55 50.84) (width 0.25) (layer "B.Cu") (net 21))
 (segment (start 48.55 50.4746) (end 48.55 50.84) (width 0.25) (layer "B.Cu") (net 21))
 (segment (start 50.2231 49.9981) (end 49.0265 49.9981) (width 0.25) (layer "B.Cu") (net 21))
 (segment (start 50.1 52.15) (end 45.85 52.15) (width 0.25) (layer "B.Cu") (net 24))
 (segment (start 45.85 52.15) (end 45.45 51.75) (width 0.25) (layer "B.Cu") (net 24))
 (segment (start 45.45 52.75) (end 45.55 52.65) (width 0.25) (layer "B.Cu") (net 23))
 (segment (start 45.55 52.65) (end 49.925 52.65) (width 0.25) (layer "B.Cu") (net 23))
 (segment (start 52.05 44.8) (end 48.45 44.8) (width 0.25) (layer "B.Cu") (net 32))
 (segment (start 54.8796 47.1704) (end 53.9527 47.1704) (width 0.25) (layer "B.Cu") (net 17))
 (segment (start 55.45 46.6) (end 54.8796 47.1704) (width 0.25) (layer "B.Cu") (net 17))
 (segment (start 51.4 50.35) (end 51.4 49.7231) (width 0.25) (layer "B.Cu") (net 17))
 (segment (start 53.9527 47.1704) (end 51.4 49.7231) (width 0.25) (layer "B.Cu") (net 17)))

